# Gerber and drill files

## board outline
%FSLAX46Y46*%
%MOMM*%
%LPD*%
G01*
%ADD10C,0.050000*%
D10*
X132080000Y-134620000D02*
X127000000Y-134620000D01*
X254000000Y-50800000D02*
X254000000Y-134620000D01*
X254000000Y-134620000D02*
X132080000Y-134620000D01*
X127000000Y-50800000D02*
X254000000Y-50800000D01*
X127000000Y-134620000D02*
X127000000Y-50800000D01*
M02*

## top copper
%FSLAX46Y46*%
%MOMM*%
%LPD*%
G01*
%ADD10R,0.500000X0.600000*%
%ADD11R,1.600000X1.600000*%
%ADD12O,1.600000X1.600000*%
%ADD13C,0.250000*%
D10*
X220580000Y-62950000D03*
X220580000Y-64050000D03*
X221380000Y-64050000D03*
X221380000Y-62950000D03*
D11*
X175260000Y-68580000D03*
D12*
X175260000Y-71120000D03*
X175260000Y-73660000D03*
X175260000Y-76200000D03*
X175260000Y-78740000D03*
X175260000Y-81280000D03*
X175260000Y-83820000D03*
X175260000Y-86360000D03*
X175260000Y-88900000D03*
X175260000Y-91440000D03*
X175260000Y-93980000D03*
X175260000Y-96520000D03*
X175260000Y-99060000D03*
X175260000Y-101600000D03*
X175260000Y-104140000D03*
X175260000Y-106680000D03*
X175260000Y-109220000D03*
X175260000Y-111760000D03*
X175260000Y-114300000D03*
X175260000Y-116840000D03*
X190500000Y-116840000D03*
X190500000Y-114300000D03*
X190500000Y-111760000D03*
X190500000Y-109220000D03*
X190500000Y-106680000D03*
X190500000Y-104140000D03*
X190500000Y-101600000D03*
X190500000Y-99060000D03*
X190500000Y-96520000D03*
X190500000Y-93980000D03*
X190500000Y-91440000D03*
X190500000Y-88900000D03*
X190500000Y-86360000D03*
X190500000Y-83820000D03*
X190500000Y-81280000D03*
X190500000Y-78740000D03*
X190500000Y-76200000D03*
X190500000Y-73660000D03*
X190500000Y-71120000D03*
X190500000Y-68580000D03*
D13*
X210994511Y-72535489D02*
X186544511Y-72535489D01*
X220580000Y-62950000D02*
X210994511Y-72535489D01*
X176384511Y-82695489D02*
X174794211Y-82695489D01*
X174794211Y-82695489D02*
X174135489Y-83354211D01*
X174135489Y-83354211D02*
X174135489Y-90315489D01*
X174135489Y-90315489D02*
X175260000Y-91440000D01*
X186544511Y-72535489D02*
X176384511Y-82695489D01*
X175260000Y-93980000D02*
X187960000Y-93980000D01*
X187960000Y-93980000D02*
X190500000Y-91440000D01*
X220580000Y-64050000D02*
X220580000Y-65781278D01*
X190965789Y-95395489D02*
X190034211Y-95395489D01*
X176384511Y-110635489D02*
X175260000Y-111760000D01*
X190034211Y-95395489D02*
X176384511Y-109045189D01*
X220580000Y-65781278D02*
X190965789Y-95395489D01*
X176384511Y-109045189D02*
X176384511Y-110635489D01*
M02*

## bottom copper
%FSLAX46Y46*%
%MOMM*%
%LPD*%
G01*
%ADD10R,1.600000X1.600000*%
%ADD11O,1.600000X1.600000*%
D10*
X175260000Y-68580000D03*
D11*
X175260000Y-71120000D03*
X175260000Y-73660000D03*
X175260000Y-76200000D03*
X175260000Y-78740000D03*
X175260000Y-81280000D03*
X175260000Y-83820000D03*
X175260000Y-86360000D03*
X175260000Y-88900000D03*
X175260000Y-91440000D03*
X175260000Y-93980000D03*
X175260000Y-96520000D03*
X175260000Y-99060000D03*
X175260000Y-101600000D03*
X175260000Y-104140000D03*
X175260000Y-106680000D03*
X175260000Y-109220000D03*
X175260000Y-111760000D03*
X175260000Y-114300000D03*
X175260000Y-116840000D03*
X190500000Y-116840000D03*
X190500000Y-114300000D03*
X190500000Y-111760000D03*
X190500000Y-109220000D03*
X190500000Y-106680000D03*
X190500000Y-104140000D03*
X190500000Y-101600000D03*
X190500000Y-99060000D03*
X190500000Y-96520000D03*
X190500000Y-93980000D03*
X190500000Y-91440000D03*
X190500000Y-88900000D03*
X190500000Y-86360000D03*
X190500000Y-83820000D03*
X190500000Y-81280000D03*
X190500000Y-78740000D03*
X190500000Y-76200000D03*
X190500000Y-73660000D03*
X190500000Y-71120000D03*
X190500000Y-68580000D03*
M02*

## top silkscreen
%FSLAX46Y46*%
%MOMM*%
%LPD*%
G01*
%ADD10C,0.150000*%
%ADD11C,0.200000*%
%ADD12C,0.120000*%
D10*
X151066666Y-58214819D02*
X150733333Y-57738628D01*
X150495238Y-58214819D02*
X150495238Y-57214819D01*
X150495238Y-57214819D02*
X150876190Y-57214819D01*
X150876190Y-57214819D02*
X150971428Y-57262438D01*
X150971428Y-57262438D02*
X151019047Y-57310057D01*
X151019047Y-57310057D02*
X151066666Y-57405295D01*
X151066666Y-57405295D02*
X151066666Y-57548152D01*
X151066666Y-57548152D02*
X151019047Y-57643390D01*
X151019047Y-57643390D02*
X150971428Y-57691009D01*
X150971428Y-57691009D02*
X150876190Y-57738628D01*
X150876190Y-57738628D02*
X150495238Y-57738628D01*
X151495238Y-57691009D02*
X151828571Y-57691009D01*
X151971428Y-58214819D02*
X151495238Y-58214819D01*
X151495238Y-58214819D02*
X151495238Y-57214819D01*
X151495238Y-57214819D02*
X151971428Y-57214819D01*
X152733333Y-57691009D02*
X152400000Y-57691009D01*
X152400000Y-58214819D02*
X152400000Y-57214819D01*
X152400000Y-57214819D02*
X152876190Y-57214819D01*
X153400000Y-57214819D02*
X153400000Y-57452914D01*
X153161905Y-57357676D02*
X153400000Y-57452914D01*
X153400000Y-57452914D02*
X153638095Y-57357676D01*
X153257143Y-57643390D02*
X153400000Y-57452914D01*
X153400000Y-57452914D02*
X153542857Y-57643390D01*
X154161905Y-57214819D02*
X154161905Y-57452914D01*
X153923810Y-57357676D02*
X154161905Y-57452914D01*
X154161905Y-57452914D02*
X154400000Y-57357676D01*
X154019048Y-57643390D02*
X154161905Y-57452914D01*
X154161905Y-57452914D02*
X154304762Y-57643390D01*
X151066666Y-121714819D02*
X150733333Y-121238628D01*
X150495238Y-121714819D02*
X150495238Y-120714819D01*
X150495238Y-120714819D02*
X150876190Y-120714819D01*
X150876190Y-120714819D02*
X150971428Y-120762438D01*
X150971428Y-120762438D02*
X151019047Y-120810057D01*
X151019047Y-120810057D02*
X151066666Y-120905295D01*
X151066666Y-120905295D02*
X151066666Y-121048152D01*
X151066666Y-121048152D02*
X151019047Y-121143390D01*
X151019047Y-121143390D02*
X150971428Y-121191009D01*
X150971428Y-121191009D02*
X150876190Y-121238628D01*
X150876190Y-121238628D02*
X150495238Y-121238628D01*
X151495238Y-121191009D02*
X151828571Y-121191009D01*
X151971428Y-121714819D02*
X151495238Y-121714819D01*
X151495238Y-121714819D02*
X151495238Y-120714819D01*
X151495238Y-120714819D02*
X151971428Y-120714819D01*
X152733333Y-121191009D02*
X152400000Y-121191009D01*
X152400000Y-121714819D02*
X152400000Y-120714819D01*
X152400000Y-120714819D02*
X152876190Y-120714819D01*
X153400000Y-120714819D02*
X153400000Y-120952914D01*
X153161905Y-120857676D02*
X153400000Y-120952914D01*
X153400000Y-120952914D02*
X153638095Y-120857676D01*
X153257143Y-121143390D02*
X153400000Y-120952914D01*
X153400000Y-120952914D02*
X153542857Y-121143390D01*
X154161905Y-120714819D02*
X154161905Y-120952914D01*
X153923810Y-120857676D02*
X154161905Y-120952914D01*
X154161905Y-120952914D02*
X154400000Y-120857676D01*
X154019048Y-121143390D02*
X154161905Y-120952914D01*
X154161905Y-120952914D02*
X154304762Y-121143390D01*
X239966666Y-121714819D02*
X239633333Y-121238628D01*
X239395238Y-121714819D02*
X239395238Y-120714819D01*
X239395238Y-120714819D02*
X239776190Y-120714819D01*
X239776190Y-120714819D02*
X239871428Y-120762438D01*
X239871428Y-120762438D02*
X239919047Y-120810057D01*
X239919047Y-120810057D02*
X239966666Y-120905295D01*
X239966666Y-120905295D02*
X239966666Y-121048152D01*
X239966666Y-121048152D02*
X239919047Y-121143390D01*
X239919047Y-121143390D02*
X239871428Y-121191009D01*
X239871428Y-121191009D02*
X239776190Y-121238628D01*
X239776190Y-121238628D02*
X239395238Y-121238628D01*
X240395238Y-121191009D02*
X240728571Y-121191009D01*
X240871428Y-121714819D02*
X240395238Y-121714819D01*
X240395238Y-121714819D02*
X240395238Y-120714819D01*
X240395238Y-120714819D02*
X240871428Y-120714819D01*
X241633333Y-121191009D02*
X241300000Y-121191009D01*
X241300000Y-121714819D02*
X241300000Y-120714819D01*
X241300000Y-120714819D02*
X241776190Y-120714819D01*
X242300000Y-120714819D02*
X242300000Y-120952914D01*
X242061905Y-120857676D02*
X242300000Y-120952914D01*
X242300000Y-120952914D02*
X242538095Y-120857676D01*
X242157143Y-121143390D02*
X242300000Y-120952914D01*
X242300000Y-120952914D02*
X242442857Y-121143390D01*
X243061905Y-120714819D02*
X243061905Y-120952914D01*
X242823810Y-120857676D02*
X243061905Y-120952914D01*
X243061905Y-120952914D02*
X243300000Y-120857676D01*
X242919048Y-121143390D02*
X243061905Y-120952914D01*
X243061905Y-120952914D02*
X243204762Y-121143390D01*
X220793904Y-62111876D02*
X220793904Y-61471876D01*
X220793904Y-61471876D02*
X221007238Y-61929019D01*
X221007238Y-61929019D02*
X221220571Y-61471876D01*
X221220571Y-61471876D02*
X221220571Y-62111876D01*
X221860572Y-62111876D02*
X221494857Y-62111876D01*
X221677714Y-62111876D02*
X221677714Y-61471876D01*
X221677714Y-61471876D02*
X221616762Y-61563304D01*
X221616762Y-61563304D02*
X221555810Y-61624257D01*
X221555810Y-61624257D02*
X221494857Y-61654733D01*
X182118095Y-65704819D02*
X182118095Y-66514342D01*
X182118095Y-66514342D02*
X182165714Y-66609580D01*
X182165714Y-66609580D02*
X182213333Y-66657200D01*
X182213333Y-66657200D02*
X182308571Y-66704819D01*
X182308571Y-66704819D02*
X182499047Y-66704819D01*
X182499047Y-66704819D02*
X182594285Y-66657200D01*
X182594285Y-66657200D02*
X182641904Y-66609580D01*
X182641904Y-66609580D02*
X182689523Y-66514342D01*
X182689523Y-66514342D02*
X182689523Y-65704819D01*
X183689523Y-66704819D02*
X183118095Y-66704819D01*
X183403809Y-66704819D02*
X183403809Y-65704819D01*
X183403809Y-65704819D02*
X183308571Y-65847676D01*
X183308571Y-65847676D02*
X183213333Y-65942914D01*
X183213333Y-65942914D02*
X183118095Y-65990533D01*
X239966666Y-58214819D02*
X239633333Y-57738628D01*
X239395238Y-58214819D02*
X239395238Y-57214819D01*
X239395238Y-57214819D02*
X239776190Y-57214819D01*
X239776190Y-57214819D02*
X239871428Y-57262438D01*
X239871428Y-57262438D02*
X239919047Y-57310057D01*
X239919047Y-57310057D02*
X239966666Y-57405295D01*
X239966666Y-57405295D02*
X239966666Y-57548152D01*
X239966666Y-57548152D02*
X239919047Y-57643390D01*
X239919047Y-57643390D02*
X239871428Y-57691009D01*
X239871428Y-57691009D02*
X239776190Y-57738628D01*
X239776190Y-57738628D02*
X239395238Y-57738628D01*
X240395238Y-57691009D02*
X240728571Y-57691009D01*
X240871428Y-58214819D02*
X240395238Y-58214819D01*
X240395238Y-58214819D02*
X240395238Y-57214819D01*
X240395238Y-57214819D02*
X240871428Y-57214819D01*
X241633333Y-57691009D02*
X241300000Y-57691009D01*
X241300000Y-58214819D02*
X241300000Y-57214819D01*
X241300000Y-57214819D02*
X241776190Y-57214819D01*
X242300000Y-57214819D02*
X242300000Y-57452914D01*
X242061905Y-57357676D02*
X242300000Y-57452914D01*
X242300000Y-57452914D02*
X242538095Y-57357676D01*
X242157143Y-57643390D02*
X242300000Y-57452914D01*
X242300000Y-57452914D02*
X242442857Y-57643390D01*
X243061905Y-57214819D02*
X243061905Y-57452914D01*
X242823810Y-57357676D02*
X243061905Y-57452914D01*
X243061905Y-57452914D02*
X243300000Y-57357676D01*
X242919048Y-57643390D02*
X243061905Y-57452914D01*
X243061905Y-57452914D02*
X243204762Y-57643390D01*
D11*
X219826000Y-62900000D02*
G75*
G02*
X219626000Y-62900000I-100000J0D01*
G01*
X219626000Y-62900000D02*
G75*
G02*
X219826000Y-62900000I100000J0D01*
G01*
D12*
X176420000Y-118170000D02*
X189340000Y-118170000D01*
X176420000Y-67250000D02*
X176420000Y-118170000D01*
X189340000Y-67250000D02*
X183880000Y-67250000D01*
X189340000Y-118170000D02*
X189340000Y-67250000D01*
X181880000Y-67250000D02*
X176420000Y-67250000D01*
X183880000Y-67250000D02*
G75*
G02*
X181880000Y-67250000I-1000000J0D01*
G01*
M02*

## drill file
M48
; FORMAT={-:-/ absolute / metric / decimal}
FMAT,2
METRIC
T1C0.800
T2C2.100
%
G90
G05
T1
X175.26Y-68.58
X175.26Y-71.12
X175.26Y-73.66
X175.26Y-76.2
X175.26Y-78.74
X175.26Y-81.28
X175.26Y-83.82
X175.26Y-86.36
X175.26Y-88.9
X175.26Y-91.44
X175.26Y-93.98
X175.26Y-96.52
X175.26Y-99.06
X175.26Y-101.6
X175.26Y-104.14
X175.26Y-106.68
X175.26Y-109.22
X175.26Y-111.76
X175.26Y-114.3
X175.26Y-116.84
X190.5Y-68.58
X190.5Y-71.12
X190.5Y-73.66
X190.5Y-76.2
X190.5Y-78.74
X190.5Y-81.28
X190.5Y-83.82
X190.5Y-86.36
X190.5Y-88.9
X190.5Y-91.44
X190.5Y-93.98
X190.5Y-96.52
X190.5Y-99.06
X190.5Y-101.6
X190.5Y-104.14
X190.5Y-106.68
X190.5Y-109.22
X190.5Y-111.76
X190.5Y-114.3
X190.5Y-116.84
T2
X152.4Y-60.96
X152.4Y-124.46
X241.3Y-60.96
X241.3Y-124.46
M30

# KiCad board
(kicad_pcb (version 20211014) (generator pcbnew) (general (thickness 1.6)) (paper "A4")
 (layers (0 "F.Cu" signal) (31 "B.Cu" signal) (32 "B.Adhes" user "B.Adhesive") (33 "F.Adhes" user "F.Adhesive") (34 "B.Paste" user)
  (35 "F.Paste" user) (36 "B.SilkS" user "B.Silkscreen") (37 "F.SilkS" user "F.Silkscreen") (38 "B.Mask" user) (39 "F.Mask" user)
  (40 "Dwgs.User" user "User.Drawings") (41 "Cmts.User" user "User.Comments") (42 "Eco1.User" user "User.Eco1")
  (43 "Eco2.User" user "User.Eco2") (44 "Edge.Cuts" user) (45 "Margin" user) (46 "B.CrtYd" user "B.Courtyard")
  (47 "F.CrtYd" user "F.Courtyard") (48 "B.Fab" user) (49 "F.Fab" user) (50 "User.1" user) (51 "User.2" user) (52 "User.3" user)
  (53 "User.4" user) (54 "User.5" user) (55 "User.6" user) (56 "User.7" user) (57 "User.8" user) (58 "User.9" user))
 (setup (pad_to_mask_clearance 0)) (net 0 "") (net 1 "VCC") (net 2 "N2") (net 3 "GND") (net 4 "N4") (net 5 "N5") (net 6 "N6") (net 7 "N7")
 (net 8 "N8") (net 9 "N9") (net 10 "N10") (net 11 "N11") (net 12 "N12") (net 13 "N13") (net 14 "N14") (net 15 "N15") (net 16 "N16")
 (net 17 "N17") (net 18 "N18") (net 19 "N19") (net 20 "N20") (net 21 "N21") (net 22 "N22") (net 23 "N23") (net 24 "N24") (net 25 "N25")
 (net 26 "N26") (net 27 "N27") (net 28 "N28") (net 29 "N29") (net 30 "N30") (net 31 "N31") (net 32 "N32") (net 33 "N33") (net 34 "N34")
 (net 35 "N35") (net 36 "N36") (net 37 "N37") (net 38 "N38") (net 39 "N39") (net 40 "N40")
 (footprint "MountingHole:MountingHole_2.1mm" (layer "F.Cu") (at 152.4 60.96)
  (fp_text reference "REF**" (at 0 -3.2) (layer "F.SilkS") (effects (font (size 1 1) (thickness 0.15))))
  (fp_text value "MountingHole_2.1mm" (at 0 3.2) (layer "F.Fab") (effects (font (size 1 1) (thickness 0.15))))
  (pad "" np_thru_hole circle (at 0 0) (size 2.1 2.1) (drill 2.1) (layers *.Cu *.Mask)))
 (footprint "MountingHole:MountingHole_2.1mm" (layer "F.Cu") (at 152.4 124.46)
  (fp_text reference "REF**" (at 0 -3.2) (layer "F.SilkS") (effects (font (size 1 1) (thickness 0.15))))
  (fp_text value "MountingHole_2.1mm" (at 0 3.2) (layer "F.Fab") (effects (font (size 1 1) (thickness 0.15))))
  (pad "" np_thru_hole circle (at 0 0) (size 2.1 2.1) (drill 2.1) (layers *.Cu *.Mask)))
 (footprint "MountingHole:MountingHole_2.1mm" (layer "F.Cu") (at 241.3 124.46)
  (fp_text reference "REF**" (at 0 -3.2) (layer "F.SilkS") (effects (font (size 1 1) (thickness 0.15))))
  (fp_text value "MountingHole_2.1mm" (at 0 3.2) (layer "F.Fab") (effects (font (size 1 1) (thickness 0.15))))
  (pad "" np_thru_hole circle (at 0 0) (size 2.1 2.1) (drill 2.1) (layers *.Cu *.Mask)))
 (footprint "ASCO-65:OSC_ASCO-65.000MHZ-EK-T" (layer "F.Cu") (at 220.98 63.5)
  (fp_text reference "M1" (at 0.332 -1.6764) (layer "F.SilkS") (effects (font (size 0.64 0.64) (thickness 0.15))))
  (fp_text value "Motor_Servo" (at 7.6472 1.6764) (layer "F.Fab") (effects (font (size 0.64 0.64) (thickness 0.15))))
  (fp_circle (center -1.254 -0.6) (end -1.154 -0.6) (layer "F.SilkS") (width 0.2) (fill none))
  (pad "1" smd rect locked (at -0.4 -0.55) (size 0.5 0.6) (layers "F.Cu" "F.Paste" "F.Mask") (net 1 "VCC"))
  (pad "2" smd rect locked (at -0.4 0.55) (size 0.5 0.6) (layers "F.Cu" "F.Paste" "F.Mask") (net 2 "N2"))
  (pad "3" smd rect locked (at 0.4 0.55) (size 0.5 0.6) (layers "F.Cu" "F.Paste" "F.Mask") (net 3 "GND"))
  (pad "4" smd rect locked (at 0.4 -0.55) (size 0.5 0.6) (layers "F.Cu" "F.Paste" "F.Mask")))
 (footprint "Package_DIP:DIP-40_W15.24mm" (layer "F.Cu") (at 175.26 68.58)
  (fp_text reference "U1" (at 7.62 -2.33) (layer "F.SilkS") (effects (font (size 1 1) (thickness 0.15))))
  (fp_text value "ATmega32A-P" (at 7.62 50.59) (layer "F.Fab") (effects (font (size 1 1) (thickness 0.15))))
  (fp_line (start 1.16 49.59) (end 14.08 49.59) (layer "F.SilkS") (width 0.12))
  (fp_line (start 1.16 -1.33) (end 1.16 49.59) (layer "F.SilkS") (width 0.12))
  (fp_line (start 14.08 -1.33) (end 8.62 -1.33) (layer "F.SilkS") (width 0.12))
  (fp_line (start 14.08 49.59) (end 14.08 -1.33) (layer "F.SilkS") (width 0.12))
  (fp_line (start 6.62 -1.33) (end 1.16 -1.33) (layer "F.SilkS") (width 0.12))
  (fp_arc (start 8.62 -1.33) (mid 7.62 -0.33) (end 6.62 -1.33) (layer "F.SilkS") (width 0.12))
  (pad "1" thru_hole rect (at 0 0) (size 1.6 1.6) (drill 0.8) (layers *.Cu *.Mask) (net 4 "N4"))
  (pad "2" thru_hole oval (at 0 2.54) (size 1.6 1.6) (drill 0.8) (layers *.Cu *.Mask) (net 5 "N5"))
  (pad "3" thru_hole oval (at 0 5.08) (size 1.6 1.6) (drill 0.8) (layers *.Cu *.Mask) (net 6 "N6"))
  (pad "4" thru_hole oval (at 0 7.62) (size 1.6 1.6) (drill 0.8) (layers *.Cu *.Mask) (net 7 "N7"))
  (pad "5" thru_hole oval (at 0 10.16) (size 1.6 1.6) (drill 0.8) (layers *.Cu *.Mask) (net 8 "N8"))
  (pad "6" thru_hole oval (at 0 12.7) (size 1.6 1.6) (drill 0.8) (layers *.Cu *.Mask) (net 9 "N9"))
  (pad "7" thru_hole oval (at 0 15.24) (size 1.6 1.6) (drill 0.8) (layers *.Cu *.Mask) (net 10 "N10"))
  (pad "8" thru_hole oval (at 0 17.78) (size 1.6 1.6) (drill 0.8) (layers *.Cu *.Mask) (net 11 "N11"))
  (pad "9" thru_hole oval (at 0 20.32) (size 1.6 1.6) (drill 0.8) (layers *.Cu *.Mask) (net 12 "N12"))
  (pad "10" thru_hole oval (at 0 22.86) (size 1.6 1.6) (drill 0.8) (layers *.Cu *.Mask) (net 1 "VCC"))
  (pad "11" thru_hole oval (at 0 25.4) (size 1.6 1.6) (drill 0.8) (layers *.Cu *.Mask) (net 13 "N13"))
  (pad "12" thru_hole oval (at 0 27.94) (size 1.6 1.6) (drill 0.8) (layers *.Cu *.Mask) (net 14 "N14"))
  (pad "13" thru_hole oval (at 0 30.48) (size 1.6 1.6) (drill 0.8) (layers *.Cu *.Mask) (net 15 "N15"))
  (pad "14" thru_hole oval (at 0 33.02) (size 1.6 1.6) (drill 0.8) (layers *.Cu *.Mask) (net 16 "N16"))
  (pad "15" thru_hole oval (at 0 35.56) (size 1.6 1.6) (drill 0.8) (layers *.Cu *.Mask) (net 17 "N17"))
  (pad "16" thru_hole oval (at 0 38.1) (size 1.6 1.6) (drill 0.8) (layers *.Cu *.Mask) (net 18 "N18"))
  (pad "17" thru_hole oval (at 0 40.64) (size 1.6 1.6) (drill 0.8) (layers *.Cu *.Mask) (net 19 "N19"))
  (pad "18" thru_hole oval (at 0 43.18) (size 1.6 1.6) (drill 0.8) (layers *.Cu *.Mask) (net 2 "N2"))
  (pad "19" thru_hole oval (at 0 45.72) (size 1.6 1.6) (drill 0.8) (layers *.Cu *.Mask) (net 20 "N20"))
  (pad "20" thru_hole oval (at 0 48.26) (size 1.6 1.6) (drill 0.8) (layers *.Cu *.Mask) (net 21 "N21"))
  (pad "21" thru_hole oval (at 15.24 48.26) (size 1.6 1.6) (drill 0.8) (layers *.Cu *.Mask) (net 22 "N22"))
  (pad "22" thru_hole oval (at 15.24 45.72) (size 1.6 1.6) (drill 0.8) (layers *.Cu *.Mask) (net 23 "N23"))
  (pad "23" thru_hole oval (at 15.24 43.18) (size 1.6 1.6) (drill 0.8) (layers *.Cu *.Mask) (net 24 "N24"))
  (pad "24" thru_hole oval (at 15.24 40.64) (size 1.6 1.6) (drill 0.8) (layers *.Cu *.Mask) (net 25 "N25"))
  (pad "25" thru_hole oval (at 15.24 38.1) (size 1.6 1.6) (drill 0.8) (layers *.Cu *.Mask) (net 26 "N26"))
  (pad "26" thru_hole oval (at 15.24 35.56) (size 1.6 1.6) (drill 0.8) (layers *.Cu *.Mask) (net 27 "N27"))
  (pad "27" thru_hole oval (at 15.24 33.02) (size 1.6 1.6) (drill 0.8) (layers *.Cu *.Mask) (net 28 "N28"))
  (pad "28" thru_hole oval (at 15.24 30.48) (size 1.6 1.6) (drill 0.8) (layers *.Cu *.Mask) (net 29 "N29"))
  (pad "29" thru_hole oval (at 15.24 27.94) (size 1.6 1.6) (drill 0.8) (layers *.Cu *.Mask) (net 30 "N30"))
  (pad "30" thru_hole oval (at 15.24 25.4) (size 1.6 1.6) (drill 0.8) (layers *.Cu *.Mask) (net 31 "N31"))
  (pad "31" thru_hole oval (at 15.24 22.86) (size 1.6 1.6) (drill 0.8) (layers *.Cu *.Mask) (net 13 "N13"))
  (pad "32" thru_hole oval (at 15.24 20.32) (size 1.6 1.6) (drill 0.8) (layers *.Cu *.Mask) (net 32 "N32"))
  (pad "33" thru_hole oval (at 15.24 17.78) (size 1.6 1.6) (drill 0.8) (layers *.Cu *.Mask) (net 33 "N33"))
  (pad "34" thru_hole oval (at 15.24 15.24) (size 1.6 1.6) (drill 0.8) (layers *.Cu *.Mask) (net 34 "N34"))
  (pad "35" thru_hole oval (at 15.24 12.7) (size 1.6 1.6) (drill 0.8) (layers *.Cu *.Mask) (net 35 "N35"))
  (pad "36" thru_hole oval (at 15.24 10.16) (size 1.6 1.6) (drill 0.8) (layers *.Cu *.Mask) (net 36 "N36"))
  (pad "37" thru_hole oval (at 15.24 7.62) (size 1.6 1.6) (drill 0.8) (layers *.Cu *.Mask) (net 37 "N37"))
  (pad "38" thru_hole oval (at 15.24 5.08) (size 1.6 1.6) (drill 0.8) (layers *.Cu *.Mask) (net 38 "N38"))
  (pad "39" thru_hole oval (at 15.24 2.54) (size 1.6 1.6) (drill 0.8) (layers *.Cu *.Mask) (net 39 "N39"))
  (pad "40" thru_hole oval (at 15.24 0) (size 1.6 1.6) (drill 0.8) (layers *.Cu *.Mask) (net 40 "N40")))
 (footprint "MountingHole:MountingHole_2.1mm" (layer "F.Cu") (at 241.3 60.96)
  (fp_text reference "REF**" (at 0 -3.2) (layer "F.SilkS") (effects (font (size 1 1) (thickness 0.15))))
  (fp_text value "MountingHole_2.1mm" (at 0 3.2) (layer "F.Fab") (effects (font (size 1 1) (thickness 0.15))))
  (pad "" np_thru_hole circle (at 0 0) (size 2.1 2.1) (drill 2.1) (layers *.Cu *.Mask)))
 (gr_line (start 132.08 134.62) (end 127 134.62) (layer "Edge.Cuts") (width 0.05))
 (gr_line (start 254 50.8) (end 254 134.62) (layer "Edge.Cuts") (width 0.05))
 (gr_line (start 254 134.62) (end 132.08 134.62) (layer "Edge.Cuts") (width 0.05))
 (gr_line (start 127 50.8) (end 254 50.8) (layer "Edge.Cuts") (width 0.05))
 (gr_line (start 127 134.62) (end 127 50.8) (layer "Edge.Cuts") (width 0.05))
 (segment (start 210.994511 72.535489) (end 186.544511 72.535489) (width 0.25) (layer "F.Cu") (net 1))
 (segment (start 220.58 62.95) (end 210.994511 72.535489) (width 0.25) (layer "F.Cu") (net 1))
 (segment (start 176.384511 82.695489) (end 174.794211 82.695489) (width 0.25) (layer "F.Cu") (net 1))
 (segment (start 174.794211 82.695489) (end 174.135489 83.354211) (width 0.25) (layer "F.Cu") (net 1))
 (segment (start 174.135489 83.354211) (end 174.135489 90.315489) (width 0.25) (layer "F.Cu") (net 1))
 (segment (start 174.135489 90.315489) (end 175.26 91.44) (width 0.25) (layer "F.Cu") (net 1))
 (segment (start 186.544511 72.535489) (end 176.384511 82.695489) (width 0.25) (layer "F.Cu") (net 1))
 (segment (start 175.26 93.98) (end 187.96 93.98) (width 0.25) (layer "F.Cu") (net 13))
 (segment (start 187.96 93.98) (end 190.5 91.44) (width 0.25) (layer "F.Cu") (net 13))
 (segment (start 220.58 64.05) (end 220.58 65.781278) (width 0.25) (layer "F.Cu") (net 2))
 (segment (start 190.965789 95.395489) (end 190.034211 95.395489) (width 0.25) (layer "F.Cu") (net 2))
 (segment (start 176.384511 110.635489) (end 175.26 111.76) (width 0.25) (layer "F.Cu") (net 2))
 (segment (start 190.034211 95.395489) (end 176.384511 109.045189) (width 0.25) (layer "F.Cu") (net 2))
 (segment (start 220.58 65.781278) (end 190.965789 95.395489) (width 0.25) (layer "F.Cu") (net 2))
 (segment (start 176.384511 109.045189) (end 176.384511 110.635489) (width 0.25) (layer "F.Cu") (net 2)))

